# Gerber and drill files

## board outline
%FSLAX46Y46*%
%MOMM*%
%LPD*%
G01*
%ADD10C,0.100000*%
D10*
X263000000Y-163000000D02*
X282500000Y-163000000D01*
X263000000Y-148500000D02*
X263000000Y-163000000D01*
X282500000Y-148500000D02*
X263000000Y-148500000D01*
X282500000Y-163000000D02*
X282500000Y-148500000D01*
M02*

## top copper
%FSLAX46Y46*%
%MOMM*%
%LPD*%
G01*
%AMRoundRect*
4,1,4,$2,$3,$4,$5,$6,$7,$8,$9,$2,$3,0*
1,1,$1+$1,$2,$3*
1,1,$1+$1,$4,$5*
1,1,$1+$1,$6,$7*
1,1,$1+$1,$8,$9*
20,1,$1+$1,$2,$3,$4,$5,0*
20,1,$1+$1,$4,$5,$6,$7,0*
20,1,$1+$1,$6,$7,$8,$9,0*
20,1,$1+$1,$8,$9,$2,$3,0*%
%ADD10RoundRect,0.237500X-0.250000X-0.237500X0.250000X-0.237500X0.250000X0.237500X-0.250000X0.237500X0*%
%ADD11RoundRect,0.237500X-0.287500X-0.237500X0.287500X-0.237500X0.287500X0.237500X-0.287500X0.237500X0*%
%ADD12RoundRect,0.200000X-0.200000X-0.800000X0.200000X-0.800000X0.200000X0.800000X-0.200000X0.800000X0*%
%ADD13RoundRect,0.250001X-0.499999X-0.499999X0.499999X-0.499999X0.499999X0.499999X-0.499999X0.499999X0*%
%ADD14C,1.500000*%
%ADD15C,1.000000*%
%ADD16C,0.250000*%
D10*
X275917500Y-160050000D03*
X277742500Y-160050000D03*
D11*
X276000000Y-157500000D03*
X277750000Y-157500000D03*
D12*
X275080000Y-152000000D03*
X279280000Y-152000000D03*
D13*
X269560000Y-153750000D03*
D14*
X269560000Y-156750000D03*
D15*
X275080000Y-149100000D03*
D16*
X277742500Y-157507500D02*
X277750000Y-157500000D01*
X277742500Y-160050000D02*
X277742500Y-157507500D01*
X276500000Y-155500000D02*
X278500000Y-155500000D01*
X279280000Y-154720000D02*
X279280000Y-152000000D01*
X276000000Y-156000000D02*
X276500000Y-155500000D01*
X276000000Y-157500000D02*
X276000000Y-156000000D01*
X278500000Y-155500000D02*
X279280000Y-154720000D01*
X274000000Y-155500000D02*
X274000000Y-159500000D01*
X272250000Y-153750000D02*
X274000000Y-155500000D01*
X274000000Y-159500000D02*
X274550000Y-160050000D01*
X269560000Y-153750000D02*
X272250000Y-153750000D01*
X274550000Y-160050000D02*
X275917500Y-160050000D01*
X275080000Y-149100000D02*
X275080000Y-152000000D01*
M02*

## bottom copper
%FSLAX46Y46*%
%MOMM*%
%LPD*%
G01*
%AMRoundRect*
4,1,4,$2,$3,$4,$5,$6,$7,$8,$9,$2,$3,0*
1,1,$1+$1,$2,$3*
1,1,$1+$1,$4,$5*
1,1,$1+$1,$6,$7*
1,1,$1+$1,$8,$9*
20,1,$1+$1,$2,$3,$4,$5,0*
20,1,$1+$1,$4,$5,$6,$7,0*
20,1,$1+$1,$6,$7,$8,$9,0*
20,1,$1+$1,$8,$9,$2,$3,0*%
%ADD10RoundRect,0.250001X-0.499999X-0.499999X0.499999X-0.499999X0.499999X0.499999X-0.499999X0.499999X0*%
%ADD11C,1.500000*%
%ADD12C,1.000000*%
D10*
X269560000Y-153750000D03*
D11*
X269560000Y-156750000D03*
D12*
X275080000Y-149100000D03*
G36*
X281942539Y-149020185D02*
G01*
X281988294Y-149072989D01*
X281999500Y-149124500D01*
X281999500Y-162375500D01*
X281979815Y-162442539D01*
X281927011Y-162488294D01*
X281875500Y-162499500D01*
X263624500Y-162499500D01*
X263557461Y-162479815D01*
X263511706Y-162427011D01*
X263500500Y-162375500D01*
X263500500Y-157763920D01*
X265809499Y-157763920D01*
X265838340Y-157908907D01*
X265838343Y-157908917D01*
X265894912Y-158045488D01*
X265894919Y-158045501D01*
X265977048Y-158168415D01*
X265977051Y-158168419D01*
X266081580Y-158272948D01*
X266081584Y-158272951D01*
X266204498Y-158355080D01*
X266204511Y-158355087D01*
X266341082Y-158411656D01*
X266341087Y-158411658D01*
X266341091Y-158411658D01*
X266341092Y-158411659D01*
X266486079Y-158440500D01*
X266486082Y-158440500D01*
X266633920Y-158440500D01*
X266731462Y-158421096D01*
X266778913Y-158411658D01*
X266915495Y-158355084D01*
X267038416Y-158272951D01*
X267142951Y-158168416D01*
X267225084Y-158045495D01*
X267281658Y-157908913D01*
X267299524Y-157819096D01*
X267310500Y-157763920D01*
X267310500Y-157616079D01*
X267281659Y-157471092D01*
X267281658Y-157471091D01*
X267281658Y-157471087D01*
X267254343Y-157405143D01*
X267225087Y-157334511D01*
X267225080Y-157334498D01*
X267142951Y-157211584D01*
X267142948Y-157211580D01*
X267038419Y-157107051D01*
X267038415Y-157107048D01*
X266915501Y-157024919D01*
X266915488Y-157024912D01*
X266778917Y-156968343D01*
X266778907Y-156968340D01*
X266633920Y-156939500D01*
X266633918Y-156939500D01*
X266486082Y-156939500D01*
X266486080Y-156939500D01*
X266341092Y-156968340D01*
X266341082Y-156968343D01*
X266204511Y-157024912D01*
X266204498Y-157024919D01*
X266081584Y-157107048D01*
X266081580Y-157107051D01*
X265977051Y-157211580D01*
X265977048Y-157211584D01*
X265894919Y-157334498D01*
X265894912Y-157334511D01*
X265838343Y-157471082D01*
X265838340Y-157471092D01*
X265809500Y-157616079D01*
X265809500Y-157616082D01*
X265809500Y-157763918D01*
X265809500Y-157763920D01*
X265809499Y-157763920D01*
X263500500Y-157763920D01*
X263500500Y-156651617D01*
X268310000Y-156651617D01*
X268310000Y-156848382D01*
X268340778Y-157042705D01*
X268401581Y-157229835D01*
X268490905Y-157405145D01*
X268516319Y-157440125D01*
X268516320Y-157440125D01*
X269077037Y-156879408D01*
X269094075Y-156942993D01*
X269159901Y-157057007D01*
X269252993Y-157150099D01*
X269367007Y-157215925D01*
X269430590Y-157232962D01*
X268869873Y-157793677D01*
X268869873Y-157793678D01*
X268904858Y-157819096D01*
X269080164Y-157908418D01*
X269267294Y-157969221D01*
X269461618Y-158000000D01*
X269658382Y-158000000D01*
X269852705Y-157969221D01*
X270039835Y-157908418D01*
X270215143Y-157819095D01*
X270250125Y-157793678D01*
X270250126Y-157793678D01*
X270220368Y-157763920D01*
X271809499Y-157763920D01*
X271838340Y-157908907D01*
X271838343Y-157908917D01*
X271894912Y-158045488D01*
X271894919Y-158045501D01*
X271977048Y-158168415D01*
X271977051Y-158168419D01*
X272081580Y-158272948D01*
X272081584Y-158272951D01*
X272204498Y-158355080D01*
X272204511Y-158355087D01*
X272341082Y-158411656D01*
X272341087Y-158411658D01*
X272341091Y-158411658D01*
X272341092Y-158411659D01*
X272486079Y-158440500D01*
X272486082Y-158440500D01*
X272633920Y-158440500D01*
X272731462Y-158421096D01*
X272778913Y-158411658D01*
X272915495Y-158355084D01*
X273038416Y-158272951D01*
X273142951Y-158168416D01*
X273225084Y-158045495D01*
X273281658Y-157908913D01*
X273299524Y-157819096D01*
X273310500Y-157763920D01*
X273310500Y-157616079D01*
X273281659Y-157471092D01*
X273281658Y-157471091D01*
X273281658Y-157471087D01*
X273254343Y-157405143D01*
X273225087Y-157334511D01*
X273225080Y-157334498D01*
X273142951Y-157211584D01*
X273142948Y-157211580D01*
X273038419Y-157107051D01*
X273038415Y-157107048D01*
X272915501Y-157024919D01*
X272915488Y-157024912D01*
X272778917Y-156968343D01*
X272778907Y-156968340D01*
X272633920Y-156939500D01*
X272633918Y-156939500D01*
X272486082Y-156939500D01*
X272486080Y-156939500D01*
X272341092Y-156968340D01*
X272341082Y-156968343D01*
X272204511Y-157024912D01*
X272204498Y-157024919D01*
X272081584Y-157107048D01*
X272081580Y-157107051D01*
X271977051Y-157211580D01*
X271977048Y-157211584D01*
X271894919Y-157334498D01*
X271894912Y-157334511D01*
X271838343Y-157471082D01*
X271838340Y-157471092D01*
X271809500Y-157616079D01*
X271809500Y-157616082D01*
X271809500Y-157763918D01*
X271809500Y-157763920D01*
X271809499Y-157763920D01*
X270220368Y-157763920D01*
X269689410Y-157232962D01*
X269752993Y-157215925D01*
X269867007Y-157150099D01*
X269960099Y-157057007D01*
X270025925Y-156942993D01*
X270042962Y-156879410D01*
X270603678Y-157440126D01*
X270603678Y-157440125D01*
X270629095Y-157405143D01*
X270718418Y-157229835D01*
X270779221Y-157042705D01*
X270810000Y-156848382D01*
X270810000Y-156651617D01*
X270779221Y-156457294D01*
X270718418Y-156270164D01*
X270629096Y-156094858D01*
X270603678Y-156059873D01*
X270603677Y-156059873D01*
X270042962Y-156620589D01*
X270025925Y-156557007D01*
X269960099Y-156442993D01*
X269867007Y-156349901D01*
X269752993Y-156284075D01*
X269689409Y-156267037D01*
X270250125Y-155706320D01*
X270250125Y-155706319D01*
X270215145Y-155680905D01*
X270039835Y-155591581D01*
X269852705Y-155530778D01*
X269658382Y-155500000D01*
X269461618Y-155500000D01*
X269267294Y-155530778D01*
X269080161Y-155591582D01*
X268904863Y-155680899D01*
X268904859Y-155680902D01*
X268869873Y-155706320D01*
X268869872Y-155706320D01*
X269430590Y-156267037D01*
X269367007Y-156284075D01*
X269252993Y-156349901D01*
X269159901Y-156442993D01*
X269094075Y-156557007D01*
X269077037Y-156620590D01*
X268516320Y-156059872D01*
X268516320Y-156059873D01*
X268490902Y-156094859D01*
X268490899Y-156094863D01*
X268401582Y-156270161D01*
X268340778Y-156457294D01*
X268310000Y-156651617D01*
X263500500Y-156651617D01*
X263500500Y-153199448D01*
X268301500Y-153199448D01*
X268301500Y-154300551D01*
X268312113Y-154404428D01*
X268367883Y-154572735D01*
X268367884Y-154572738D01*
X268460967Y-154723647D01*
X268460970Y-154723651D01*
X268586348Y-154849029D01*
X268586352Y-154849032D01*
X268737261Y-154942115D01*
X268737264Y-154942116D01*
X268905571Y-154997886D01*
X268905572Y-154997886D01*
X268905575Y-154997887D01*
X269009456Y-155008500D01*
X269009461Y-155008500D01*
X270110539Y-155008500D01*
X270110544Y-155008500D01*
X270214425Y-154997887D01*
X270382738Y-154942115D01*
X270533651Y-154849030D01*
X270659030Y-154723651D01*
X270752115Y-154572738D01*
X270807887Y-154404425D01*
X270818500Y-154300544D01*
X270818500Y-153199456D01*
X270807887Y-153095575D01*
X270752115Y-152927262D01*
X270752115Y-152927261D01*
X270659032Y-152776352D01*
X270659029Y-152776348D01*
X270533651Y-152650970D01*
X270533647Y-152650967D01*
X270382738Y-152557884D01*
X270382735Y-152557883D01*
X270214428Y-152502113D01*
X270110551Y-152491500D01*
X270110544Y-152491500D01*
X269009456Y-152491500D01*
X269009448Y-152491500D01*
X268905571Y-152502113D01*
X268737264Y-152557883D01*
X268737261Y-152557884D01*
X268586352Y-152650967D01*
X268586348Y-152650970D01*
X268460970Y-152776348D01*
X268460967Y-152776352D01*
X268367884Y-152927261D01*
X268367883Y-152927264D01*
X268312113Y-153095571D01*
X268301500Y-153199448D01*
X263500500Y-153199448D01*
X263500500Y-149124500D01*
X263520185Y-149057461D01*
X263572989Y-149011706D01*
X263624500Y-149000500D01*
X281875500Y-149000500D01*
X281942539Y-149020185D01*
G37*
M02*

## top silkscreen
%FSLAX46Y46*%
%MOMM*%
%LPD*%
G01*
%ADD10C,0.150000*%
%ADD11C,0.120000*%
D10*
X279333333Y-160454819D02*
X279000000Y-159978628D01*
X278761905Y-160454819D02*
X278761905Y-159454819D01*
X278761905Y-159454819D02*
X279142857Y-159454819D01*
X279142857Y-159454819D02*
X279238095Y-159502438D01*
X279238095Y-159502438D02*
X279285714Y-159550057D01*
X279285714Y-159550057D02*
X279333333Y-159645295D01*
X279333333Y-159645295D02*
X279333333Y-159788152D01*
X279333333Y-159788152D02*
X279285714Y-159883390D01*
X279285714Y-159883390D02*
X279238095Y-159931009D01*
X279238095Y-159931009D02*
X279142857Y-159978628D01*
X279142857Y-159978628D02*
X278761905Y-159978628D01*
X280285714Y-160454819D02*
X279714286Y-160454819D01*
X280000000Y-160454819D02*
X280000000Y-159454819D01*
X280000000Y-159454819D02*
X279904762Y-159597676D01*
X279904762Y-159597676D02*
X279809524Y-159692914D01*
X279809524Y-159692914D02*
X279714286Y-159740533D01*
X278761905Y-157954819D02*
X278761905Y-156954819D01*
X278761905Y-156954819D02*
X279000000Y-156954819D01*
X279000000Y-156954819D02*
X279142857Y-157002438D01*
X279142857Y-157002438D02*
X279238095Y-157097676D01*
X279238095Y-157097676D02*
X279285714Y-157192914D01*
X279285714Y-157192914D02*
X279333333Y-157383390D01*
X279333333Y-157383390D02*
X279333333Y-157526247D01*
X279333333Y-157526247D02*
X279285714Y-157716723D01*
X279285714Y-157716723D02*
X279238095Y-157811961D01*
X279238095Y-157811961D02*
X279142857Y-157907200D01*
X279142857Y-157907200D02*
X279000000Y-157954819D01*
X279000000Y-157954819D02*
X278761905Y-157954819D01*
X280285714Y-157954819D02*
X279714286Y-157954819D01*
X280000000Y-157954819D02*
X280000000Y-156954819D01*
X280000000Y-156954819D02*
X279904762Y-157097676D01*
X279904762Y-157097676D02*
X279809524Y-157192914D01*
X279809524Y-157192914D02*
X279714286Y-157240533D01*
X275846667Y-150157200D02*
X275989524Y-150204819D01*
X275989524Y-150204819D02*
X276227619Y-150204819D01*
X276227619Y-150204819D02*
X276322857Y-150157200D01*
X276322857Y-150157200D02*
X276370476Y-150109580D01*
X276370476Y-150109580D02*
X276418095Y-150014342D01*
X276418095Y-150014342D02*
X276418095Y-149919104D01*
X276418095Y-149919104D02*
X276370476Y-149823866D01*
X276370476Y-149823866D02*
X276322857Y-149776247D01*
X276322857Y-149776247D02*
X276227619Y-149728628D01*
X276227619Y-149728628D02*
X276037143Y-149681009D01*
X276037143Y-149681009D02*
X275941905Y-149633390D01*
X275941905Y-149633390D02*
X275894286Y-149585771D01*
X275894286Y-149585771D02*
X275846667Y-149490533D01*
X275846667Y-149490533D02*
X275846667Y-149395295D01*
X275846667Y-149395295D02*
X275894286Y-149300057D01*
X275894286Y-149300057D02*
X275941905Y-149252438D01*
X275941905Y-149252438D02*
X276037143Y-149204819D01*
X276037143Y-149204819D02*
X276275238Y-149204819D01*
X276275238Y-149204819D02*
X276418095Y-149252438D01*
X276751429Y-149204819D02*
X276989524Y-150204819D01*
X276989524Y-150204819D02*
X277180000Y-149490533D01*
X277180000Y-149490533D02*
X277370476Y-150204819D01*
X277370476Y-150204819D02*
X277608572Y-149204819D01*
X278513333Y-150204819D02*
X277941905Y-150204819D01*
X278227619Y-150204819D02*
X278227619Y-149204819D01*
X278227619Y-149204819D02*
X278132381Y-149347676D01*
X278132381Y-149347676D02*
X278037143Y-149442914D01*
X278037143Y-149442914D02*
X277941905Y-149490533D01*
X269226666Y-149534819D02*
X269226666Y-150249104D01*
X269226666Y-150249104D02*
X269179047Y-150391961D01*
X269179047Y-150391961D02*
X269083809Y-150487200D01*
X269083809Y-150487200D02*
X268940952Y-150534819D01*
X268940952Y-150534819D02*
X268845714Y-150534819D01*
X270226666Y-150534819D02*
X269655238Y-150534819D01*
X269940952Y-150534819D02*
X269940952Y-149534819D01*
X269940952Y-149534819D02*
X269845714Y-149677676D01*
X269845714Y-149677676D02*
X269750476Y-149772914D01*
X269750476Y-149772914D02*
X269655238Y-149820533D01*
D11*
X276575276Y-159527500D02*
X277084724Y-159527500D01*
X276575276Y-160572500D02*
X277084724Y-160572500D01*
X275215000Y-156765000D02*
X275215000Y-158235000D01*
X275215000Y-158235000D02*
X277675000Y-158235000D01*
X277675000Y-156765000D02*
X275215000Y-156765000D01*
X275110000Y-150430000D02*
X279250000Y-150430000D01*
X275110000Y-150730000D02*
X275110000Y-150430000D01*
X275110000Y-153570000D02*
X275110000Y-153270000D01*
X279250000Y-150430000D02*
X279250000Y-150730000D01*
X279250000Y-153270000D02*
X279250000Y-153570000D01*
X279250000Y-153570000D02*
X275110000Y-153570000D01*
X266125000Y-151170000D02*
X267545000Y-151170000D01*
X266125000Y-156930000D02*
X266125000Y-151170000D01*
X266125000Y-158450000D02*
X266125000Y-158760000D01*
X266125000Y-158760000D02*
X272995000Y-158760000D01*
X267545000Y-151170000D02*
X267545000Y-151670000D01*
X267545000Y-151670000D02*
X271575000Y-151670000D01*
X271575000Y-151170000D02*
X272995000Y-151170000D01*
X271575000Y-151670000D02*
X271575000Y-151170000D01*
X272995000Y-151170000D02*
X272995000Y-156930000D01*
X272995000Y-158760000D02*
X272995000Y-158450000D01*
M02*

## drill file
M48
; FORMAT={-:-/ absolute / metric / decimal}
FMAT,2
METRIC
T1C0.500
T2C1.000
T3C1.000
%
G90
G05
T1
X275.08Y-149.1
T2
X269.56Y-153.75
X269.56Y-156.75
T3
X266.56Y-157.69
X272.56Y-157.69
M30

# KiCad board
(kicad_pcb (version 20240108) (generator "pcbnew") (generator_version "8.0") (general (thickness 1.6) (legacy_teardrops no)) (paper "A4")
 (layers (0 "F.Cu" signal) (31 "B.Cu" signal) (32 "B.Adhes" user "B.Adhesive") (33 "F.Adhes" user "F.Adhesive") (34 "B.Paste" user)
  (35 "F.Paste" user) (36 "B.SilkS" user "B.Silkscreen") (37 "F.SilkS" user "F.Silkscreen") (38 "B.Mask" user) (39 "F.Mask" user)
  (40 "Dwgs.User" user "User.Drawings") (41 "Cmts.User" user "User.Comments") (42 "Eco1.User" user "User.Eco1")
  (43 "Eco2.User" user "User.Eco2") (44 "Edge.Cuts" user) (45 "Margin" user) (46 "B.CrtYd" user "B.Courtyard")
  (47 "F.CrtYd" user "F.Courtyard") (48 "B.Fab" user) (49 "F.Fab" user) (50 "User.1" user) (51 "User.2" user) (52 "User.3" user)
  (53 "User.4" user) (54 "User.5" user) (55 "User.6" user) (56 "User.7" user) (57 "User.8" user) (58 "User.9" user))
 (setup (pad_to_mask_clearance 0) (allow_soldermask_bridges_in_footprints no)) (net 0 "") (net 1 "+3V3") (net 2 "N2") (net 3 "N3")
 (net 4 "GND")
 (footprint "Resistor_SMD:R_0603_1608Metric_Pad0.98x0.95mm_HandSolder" (layer "F.Cu") (at 276.83 160.05)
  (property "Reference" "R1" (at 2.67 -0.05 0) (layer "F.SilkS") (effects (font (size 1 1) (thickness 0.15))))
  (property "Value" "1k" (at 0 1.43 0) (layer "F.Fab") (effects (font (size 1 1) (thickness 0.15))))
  (fp_line (start -0.254724 -0.5225) (end 0.254724 -0.5225) (stroke (width 0.12) (type solid)) (layer "F.SilkS"))
  (fp_line (start -0.254724 0.5225) (end 0.254724 0.5225) (stroke (width 0.12) (type solid)) (layer "F.SilkS"))
  (pad "1" smd roundrect (at -0.9125 0) (size 0.975 0.95) (layers "F.Cu" "F.Paste" "F.Mask") (roundrect_rratio 0.25) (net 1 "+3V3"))
  (pad "2" smd roundrect (at 0.9125 0) (size 0.975 0.95) (layers "F.Cu" "F.Paste" "F.Mask") (roundrect_rratio 0.25) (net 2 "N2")))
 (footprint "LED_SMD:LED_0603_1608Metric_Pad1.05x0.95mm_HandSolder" (layer "F.Cu") (at 276.875 157.5)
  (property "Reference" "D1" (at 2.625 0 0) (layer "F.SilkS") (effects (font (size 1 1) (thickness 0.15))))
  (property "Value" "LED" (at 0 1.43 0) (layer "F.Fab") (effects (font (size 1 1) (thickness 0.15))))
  (fp_line (start -1.66 -0.735) (end -1.66 0.735) (stroke (width 0.12) (type solid)) (layer "F.SilkS"))
  (fp_line (start -1.66 0.735) (end 0.8 0.735) (stroke (width 0.12) (type solid)) (layer "F.SilkS"))
  (fp_line (start 0.8 -0.735) (end -1.66 -0.735) (stroke (width 0.12) (type solid)) (layer "F.SilkS"))
  (pad "1" smd roundrect (at -0.875 0) (size 1.05 0.95) (layers "F.Cu" "F.Paste" "F.Mask") (roundrect_rratio 0.25) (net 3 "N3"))
  (pad "2" smd roundrect (at 0.875 0) (size 1.05 0.95) (layers "F.Cu" "F.Paste" "F.Mask") (roundrect_rratio 0.25) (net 2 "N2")))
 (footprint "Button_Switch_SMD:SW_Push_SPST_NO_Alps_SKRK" (layer "F.Cu") (at 277.18 152)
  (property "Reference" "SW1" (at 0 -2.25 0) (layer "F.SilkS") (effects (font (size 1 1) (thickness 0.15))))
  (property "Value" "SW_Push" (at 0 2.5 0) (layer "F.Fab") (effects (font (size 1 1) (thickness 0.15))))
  (fp_line (start -2.07 -1.57) (end 2.07 -1.57) (stroke (width 0.12) (type solid)) (layer "F.SilkS"))
  (fp_line (start -2.07 -1.27) (end -2.07 -1.57) (stroke (width 0.12) (type solid)) (layer "F.SilkS"))
  (fp_line (start -2.07 1.57) (end -2.07 1.27) (stroke (width 0.12) (type solid)) (layer "F.SilkS"))
  (fp_line (start 2.07 -1.57) (end 2.07 -1.27) (stroke (width 0.12) (type solid)) (layer "F.SilkS"))
  (fp_line (start 2.07 1.27) (end 2.07 1.57) (stroke (width 0.12) (type solid)) (layer "F.SilkS"))
  (fp_line (start 2.07 1.57) (end -2.07 1.57) (stroke (width 0.12) (type solid)) (layer "F.SilkS"))
  (pad "1" smd roundrect (at -2.1 0) (size 0.8 2) (layers "F.Cu" "F.Paste" "F.Mask") (roundrect_rratio 0.25) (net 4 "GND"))
  (pad "2" smd roundrect (at 2.1 0) (size 0.8 2) (layers "F.Cu" "F.Paste" "F.Mask") (roundrect_rratio 0.25) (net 3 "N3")))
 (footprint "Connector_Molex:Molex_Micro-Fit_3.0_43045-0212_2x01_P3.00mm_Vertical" (layer "F.Cu") (at 269.56 153.75)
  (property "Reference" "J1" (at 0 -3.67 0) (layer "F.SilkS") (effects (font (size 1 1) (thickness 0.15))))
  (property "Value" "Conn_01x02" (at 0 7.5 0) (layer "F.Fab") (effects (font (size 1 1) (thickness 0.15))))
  (fp_line (start -3.435 -2.58) (end -2.015 -2.58) (stroke (width 0.12) (type solid)) (layer "F.SilkS"))
  (fp_line (start -3.435 3.18) (end -3.435 -2.58) (stroke (width 0.12) (type solid)) (layer "F.SilkS"))
  (fp_line (start -3.435 4.7) (end -3.435 5.01) (stroke (width 0.12) (type solid)) (layer "F.SilkS"))
  (fp_line (start -3.435 5.01) (end 3.435 5.01) (stroke (width 0.12) (type solid)) (layer "F.SilkS"))
  (fp_line (start -2.015 -2.58) (end -2.015 -2.08) (stroke (width 0.12) (type solid)) (layer "F.SilkS"))
  (fp_line (start -2.015 -2.08) (end 2.015 -2.08) (stroke (width 0.12) (type solid)) (layer "F.SilkS"))
  (fp_line (start 2.015 -2.58) (end 3.435 -2.58) (stroke (width 0.12) (type solid)) (layer "F.SilkS"))
  (fp_line (start 2.015 -2.08) (end 2.015 -2.58) (stroke (width 0.12) (type solid)) (layer "F.SilkS"))
  (fp_line (start 3.435 -2.58) (end 3.435 3.18) (stroke (width 0.12) (type solid)) (layer "F.SilkS"))
  (fp_line (start 3.435 5.01) (end 3.435 4.7) (stroke (width 0.12) (type solid)) (layer "F.SilkS"))
  (pad "" np_thru_hole circle (at -3 3.94) (size 1 1) (drill 1) (layers "*.Cu" "*.Mask"))
  (pad "" np_thru_hole circle (at 3 3.94) (size 1 1) (drill 1) (layers "*.Cu" "*.Mask"))
  (pad "1" thru_hole roundrect (at 0 0) (size 1.5 1.5) (drill 1) (layers "*.Cu" "*.Mask") (remove_unused_layers no)
   (roundrect_rratio 0.166667) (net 1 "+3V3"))
  (pad "2" thru_hole circle (at 0 3) (size 1.5 1.5) (drill 1) (layers "*.Cu" "*.Mask") (remove_unused_layers no) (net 4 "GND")))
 (gr_line (start 263 163) (end 282.5 163) (stroke (width 0.1) (type default)) (layer "Edge.Cuts"))
 (gr_line (start 263 148.5) (end 263 163) (stroke (width 0.1) (type default)) (layer "Edge.Cuts"))
 (gr_line (start 282.5 148.5) (end 263 148.5) (stroke (width 0.1) (type default)) (layer "Edge.Cuts"))
 (gr_line (start 282.5 163) (end 282.5 148.5) (stroke (width 0.1) (type default)) (layer "Edge.Cuts"))
 (segment (start 277.7425 157.5075) (end 277.75 157.5) (width 0.25) (layer "F.Cu") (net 2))
 (segment (start 277.7425 160.05) (end 277.7425 157.5075) (width 0.25) (layer "F.Cu") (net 2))
 (segment (start 276.5 155.5) (end 278.5 155.5) (width 0.25) (layer "F.Cu") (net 3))
 (segment (start 279.28 154.72) (end 279.28 152) (width 0.25) (layer "F.Cu") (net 3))
 (segment (start 276 156) (end 276.5 155.5) (width 0.25) (layer "F.Cu") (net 3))
 (segment (start 276 157.5) (end 276 156) (width 0.25) (layer "F.Cu") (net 3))
 (segment (start 278.5 155.5) (end 279.28 154.72) (width 0.25) (layer "F.Cu") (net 3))
 (segment (start 274 155.5) (end 274 159.5) (width 0.25) (layer "F.Cu") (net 1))
 (segment (start 272.25 153.75) (end 274 155.5) (width 0.25) (layer "F.Cu") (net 1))
 (segment (start 274 159.5) (end 274.55 160.05) (width 0.25) (layer "F.Cu") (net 1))
 (segment (start 269.56 153.75) (end 272.25 153.75) (width 0.25) (layer "F.Cu") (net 1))
 (segment (start 274.55 160.05) (end 275.9175 160.05) (width 0.25) (layer "F.Cu") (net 1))
 (segment (start 275.08 149.1) (end 275.08 152) (width 0.25) (layer "F.Cu") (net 4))
 (via (at 275.08 149.1) (size 1) (drill 0.5) (layers "F.Cu" "B.Cu") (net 4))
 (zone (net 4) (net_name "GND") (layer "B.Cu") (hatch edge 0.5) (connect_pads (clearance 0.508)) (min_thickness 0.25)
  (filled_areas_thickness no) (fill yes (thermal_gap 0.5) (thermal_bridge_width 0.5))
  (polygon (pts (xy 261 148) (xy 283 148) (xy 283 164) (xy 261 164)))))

